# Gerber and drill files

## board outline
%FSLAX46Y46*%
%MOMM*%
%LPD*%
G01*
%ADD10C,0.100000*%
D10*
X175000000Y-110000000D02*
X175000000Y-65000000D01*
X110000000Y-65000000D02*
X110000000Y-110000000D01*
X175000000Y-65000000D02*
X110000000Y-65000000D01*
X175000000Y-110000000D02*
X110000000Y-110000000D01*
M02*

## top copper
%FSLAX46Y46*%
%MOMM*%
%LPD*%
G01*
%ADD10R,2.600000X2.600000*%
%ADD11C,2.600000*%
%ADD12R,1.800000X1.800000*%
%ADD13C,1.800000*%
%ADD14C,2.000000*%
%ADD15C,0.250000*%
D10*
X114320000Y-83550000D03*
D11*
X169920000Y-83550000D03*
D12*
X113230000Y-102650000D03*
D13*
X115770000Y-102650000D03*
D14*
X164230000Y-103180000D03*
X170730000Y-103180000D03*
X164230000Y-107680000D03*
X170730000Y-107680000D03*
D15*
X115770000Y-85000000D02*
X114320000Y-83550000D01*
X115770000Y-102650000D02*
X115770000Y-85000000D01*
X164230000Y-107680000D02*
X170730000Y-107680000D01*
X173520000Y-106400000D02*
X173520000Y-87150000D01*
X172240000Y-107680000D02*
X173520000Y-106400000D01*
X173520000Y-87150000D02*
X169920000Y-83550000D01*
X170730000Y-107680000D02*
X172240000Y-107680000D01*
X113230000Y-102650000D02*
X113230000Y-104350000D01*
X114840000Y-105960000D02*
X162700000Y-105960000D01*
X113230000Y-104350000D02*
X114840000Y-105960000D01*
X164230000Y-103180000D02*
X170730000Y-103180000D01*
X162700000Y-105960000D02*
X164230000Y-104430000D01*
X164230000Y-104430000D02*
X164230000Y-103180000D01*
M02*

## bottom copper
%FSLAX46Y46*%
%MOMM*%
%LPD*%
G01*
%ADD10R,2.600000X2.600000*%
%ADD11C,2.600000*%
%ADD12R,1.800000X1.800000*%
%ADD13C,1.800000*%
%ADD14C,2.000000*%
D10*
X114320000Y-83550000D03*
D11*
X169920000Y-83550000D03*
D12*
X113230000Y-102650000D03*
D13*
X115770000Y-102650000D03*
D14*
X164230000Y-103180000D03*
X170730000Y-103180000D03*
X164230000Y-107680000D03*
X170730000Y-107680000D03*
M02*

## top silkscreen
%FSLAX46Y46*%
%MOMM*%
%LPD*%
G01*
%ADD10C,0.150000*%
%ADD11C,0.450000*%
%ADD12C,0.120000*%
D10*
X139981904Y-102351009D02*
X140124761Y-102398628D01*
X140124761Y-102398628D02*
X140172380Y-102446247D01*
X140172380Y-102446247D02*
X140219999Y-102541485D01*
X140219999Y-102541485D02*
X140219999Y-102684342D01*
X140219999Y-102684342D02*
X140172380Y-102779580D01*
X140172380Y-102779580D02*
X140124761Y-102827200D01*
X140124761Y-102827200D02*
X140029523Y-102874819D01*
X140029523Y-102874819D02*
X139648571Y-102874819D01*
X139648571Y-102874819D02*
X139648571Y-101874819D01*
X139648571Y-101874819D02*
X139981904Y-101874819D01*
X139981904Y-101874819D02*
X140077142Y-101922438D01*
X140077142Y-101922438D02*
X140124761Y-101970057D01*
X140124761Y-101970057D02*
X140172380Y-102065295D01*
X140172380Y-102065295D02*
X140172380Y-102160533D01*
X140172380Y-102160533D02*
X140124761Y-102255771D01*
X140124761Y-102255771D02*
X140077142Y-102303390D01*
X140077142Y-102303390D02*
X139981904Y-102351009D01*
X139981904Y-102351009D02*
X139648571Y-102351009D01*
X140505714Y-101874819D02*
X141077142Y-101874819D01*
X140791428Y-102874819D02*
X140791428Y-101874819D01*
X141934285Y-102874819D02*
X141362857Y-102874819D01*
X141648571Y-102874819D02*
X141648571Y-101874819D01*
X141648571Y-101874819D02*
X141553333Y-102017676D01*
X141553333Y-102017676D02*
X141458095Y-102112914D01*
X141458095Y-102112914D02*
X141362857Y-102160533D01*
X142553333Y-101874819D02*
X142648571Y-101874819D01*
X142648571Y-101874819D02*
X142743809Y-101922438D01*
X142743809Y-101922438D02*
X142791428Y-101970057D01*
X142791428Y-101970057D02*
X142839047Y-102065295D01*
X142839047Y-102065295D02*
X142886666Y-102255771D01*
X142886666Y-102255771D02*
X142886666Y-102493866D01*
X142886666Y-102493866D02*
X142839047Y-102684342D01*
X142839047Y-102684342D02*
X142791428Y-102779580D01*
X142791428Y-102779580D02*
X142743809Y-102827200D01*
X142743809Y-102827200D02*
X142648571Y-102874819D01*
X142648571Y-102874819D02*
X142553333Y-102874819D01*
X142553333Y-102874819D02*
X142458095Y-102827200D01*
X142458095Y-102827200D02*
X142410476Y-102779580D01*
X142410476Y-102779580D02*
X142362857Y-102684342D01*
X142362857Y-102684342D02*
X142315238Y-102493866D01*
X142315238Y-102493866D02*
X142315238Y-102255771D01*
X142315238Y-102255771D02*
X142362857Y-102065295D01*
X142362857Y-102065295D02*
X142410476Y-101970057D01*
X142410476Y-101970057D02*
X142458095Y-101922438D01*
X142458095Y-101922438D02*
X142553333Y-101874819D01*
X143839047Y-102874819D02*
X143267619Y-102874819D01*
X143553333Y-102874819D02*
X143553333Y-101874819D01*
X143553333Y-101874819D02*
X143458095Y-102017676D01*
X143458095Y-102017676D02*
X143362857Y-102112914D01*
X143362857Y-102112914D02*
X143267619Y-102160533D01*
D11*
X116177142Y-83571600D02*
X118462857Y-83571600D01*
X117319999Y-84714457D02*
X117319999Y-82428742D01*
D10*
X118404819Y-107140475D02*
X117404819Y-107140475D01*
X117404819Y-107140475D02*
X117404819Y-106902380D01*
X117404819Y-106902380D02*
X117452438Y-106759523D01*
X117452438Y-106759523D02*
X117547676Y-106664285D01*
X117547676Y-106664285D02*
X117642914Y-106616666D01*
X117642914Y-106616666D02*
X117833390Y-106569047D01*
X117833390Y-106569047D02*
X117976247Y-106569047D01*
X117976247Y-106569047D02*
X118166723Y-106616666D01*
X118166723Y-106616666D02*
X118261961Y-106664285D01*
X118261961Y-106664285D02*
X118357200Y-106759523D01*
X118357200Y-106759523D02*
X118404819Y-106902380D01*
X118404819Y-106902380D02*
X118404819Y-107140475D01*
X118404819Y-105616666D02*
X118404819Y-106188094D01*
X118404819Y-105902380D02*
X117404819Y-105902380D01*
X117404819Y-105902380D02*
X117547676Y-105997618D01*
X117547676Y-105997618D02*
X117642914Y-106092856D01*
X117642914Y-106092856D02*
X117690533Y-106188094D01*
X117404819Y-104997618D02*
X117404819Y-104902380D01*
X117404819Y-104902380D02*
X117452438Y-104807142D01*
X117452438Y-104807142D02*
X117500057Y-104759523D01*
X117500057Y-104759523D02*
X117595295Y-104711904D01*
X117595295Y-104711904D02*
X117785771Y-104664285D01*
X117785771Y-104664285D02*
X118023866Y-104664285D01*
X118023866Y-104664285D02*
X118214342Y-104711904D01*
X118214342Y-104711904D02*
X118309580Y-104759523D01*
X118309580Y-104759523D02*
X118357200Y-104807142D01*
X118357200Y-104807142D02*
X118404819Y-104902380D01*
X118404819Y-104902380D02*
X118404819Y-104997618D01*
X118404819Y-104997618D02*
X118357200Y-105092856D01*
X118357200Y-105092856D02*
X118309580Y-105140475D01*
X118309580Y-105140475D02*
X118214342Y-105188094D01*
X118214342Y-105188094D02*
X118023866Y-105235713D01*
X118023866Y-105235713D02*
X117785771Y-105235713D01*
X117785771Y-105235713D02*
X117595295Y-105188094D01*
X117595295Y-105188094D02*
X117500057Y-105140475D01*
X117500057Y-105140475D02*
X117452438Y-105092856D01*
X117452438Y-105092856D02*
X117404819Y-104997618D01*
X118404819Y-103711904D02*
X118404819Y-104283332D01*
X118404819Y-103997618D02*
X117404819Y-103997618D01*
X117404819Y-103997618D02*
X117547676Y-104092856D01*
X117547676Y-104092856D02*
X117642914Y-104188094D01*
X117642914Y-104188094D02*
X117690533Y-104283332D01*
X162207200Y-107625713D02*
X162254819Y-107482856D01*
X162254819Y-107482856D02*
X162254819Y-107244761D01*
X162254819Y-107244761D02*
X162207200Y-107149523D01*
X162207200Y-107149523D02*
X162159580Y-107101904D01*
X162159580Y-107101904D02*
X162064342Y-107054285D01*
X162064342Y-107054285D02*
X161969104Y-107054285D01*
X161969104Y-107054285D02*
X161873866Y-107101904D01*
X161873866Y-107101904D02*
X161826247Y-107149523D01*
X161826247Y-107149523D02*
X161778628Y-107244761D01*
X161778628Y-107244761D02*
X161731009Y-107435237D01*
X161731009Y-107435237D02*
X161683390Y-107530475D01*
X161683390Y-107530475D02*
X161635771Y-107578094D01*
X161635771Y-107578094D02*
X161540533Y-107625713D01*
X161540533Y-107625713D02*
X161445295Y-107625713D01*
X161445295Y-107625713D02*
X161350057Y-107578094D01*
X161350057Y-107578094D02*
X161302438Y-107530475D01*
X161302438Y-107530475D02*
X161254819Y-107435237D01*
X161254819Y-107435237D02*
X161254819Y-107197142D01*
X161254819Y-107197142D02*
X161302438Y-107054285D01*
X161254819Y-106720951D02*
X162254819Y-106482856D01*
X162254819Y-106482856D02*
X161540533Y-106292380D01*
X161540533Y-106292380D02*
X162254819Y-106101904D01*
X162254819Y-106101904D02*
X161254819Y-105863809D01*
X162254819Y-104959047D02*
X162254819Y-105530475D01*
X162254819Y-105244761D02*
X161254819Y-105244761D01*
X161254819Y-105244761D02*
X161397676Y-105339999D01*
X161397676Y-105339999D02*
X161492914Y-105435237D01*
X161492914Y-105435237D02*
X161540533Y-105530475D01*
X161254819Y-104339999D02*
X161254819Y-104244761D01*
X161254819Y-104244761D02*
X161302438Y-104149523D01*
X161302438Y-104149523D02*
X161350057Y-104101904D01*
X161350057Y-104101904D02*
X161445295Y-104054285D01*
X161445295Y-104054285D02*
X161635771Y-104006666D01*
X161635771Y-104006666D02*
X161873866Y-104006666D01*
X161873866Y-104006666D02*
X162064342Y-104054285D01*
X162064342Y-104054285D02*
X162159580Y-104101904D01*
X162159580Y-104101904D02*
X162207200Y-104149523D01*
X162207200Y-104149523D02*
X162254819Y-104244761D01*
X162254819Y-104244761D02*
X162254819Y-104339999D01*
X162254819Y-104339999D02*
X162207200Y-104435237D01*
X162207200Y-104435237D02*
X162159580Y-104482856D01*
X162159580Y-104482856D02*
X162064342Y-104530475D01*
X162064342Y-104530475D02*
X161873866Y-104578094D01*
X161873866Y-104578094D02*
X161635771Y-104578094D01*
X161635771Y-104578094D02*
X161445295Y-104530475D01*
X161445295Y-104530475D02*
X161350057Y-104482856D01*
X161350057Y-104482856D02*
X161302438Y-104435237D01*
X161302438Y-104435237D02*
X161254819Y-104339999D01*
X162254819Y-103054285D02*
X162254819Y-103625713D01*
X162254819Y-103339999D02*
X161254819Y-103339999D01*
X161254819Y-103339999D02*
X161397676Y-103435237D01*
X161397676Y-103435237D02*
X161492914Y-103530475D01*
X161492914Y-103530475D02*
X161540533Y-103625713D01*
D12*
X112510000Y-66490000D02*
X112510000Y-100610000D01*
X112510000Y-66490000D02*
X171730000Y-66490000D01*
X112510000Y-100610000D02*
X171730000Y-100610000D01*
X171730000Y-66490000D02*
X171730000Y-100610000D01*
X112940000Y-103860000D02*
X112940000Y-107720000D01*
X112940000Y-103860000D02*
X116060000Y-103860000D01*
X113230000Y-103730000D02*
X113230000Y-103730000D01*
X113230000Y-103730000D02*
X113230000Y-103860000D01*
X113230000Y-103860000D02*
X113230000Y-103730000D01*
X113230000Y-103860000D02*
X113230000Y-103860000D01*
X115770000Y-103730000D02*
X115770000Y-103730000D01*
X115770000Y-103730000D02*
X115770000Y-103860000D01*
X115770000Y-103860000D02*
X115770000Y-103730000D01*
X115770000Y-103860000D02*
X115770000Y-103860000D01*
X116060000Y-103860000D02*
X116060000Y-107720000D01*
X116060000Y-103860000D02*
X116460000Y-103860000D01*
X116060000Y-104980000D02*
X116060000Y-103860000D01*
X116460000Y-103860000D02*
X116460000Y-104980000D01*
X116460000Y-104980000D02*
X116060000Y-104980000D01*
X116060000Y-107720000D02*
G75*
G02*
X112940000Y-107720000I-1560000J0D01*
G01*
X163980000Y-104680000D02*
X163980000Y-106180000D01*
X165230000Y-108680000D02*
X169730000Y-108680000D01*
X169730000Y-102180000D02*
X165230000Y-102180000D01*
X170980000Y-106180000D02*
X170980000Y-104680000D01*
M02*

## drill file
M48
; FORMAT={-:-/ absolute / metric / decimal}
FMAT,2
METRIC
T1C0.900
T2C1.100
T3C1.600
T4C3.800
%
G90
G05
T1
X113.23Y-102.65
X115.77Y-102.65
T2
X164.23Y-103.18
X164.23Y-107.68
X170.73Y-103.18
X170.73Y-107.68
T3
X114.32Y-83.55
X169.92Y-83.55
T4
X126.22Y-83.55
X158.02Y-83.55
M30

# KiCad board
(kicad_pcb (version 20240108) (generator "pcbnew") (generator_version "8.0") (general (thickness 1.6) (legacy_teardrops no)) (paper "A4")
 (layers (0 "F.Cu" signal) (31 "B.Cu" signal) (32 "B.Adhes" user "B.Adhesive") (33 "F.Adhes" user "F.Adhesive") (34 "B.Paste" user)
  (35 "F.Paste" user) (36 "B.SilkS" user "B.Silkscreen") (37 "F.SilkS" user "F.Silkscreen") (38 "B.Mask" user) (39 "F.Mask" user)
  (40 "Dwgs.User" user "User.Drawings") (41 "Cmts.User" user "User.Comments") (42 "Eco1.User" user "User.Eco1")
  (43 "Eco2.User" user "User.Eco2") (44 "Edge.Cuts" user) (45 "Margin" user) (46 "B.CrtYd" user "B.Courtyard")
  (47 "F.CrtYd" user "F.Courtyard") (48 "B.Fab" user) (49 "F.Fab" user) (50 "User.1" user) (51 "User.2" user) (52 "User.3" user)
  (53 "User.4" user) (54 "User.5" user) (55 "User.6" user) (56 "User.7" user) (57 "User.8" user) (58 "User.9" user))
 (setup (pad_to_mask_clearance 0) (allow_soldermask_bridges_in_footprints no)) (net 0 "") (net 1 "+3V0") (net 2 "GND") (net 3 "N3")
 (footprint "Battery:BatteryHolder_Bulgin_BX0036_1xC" (layer "F.Cu") (at 114.32 83.55)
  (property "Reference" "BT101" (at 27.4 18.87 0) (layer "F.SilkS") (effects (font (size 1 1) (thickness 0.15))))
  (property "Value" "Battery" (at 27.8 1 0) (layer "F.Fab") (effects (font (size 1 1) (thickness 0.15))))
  (fp_line (start -1.81 -17.06) (end -1.81 17.06) (stroke (width 0.12) (type solid)) (layer "F.SilkS"))
  (fp_line (start -1.81 -17.06) (end 57.41 -17.06) (stroke (width 0.12) (type solid)) (layer "F.SilkS"))
  (fp_line (start -1.81 17.06) (end 57.41 17.06) (stroke (width 0.12) (type solid)) (layer "F.SilkS"))
  (fp_line (start 57.41 -17.06) (end 57.41 17.06) (stroke (width 0.12) (type solid)) (layer "F.SilkS"))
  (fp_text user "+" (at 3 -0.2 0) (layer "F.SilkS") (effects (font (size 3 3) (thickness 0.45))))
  (pad "" np_thru_hole circle (at 11.9 0) (size 3.8 3.8) (drill 3.8) (layers "*.Cu" "*.Mask"))
  (pad "" np_thru_hole circle (at 43.7 0) (size 3.8 3.8) (drill 3.8) (layers "*.Cu" "*.Mask"))
  (pad "1" thru_hole rect (at 0 0) (size 2.6 2.6) (drill 1.6) (layers "*.Cu" "*.Mask") (remove_unused_layers no) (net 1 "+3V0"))
  (pad "2" thru_hole circle (at 55.6 0) (size 2.6 2.6) (drill 1.6) (layers "*.Cu" "*.Mask") (remove_unused_layers no) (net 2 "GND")))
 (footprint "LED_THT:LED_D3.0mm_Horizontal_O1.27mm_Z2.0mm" (layer "F.Cu") (at 113.23 102.65)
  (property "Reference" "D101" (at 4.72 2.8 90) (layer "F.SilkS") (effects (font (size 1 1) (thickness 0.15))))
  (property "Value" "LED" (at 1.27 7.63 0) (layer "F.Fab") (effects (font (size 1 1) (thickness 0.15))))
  (fp_line (start -0.29 1.21) (end -0.29 5.07) (stroke (width 0.12) (type solid)) (layer "F.SilkS"))
  (fp_line (start -0.29 1.21) (end 2.83 1.21) (stroke (width 0.12) (type solid)) (layer "F.SilkS"))
  (fp_line (start 0 1.08) (end 0 1.08) (stroke (width 0.12) (type solid)) (layer "F.SilkS"))
  (fp_line (start 0 1.08) (end 0 1.21) (stroke (width 0.12) (type solid)) (layer "F.SilkS"))
  (fp_line (start 0 1.21) (end 0 1.08) (stroke (width 0.12) (type solid)) (layer "F.SilkS"))
  (fp_line (start 0 1.21) (end 0 1.21) (stroke (width 0.12) (type solid)) (layer "F.SilkS"))
  (fp_line (start 2.54 1.08) (end 2.54 1.08) (stroke (width 0.12) (type solid)) (layer "F.SilkS"))
  (fp_line (start 2.54 1.08) (end 2.54 1.21) (stroke (width 0.12) (type solid)) (layer "F.SilkS"))
  (fp_line (start 2.54 1.21) (end 2.54 1.08) (stroke (width 0.12) (type solid)) (layer "F.SilkS"))
  (fp_line (start 2.54 1.21) (end 2.54 1.21) (stroke (width 0.12) (type solid)) (layer "F.SilkS"))
  (fp_line (start 2.83 1.21) (end 2.83 5.07) (stroke (width 0.12) (type solid)) (layer "F.SilkS"))
  (fp_line (start 2.83 1.21) (end 3.23 1.21) (stroke (width 0.12) (type solid)) (layer "F.SilkS"))
  (fp_line (start 2.83 2.33) (end 2.83 1.21) (stroke (width 0.12) (type solid)) (layer "F.SilkS"))
  (fp_line (start 3.23 1.21) (end 3.23 2.33) (stroke (width 0.12) (type solid)) (layer "F.SilkS"))
  (fp_line (start 3.23 2.33) (end 2.83 2.33) (stroke (width 0.12) (type solid)) (layer "F.SilkS"))
  (fp_arc (start 2.83 5.07) (mid 1.27 6.63) (end -0.29 5.07) (stroke (width 0.12) (type solid)) (layer "F.SilkS"))
  (pad "1" thru_hole rect (at 0 0) (size 1.8 1.8) (drill 0.9) (layers "*.Cu" "*.Mask") (remove_unused_layers no) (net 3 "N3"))
  (pad "2" thru_hole circle (at 2.54 0) (size 1.8 1.8) (drill 0.9) (layers "*.Cu" "*.Mask") (remove_unused_layers no) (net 1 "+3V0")))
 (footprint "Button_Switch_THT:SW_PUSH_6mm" (layer "F.Cu") (at 164.23 103.18)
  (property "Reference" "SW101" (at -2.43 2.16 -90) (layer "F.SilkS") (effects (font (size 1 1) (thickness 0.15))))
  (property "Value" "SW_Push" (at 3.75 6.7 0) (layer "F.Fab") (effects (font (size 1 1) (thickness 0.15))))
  (fp_line (start -0.25 1.5) (end -0.25 3) (stroke (width 0.12) (type solid)) (layer "F.SilkS"))
  (fp_line (start 1 5.5) (end 5.5 5.5) (stroke (width 0.12) (type solid)) (layer "F.SilkS"))
  (fp_line (start 5.5 -1) (end 1 -1) (stroke (width 0.12) (type solid)) (layer "F.SilkS"))
  (fp_line (start 6.75 3) (end 6.75 1.5) (stroke (width 0.12) (type solid)) (layer "F.SilkS"))
  (pad "1" thru_hole circle (at 0 0 90) (size 2 2) (drill 1.1) (layers "*.Cu" "*.Mask") (remove_unused_layers no) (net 3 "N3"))
  (pad "1" thru_hole circle (at 6.5 0 90) (size 2 2) (drill 1.1) (layers "*.Cu" "*.Mask") (remove_unused_layers no) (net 3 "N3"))
  (pad "2" thru_hole circle (at 0 4.5 90) (size 2 2) (drill 1.1) (layers "*.Cu" "*.Mask") (remove_unused_layers no) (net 2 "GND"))
  (pad "2" thru_hole circle (at 6.5 4.5 90) (size 2 2) (drill 1.1) (layers "*.Cu" "*.Mask") (remove_unused_layers no) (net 2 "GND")))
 (gr_line (start 175 110) (end 175 65) (stroke (width 0.1) (type default)) (layer "Edge.Cuts"))
 (gr_line (start 110 65) (end 110 110) (stroke (width 0.1) (type default)) (layer "Edge.Cuts"))
 (gr_line (start 175 65) (end 110 65) (stroke (width 0.1) (type default)) (layer "Edge.Cuts"))
 (gr_line (start 175 110) (end 110 110) (stroke (width 0.1) (type default)) (layer "Edge.Cuts"))
 (segment (start 115.77 85) (end 114.32 83.55) (width 0.25) (layer "F.Cu") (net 1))
 (segment (start 115.77 102.65) (end 115.77 85) (width 0.25) (layer "F.Cu") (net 1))
 (segment (start 164.23 107.68) (end 170.73 107.68) (width 0.25) (layer "F.Cu") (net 2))
 (segment (start 173.52 106.4) (end 173.52 87.15) (width 0.25) (layer "F.Cu") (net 2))
 (segment (start 172.24 107.68) (end 173.52 106.4) (width 0.25) (layer "F.Cu") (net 2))
 (segment (start 173.52 87.15) (end 169.92 83.55) (width 0.25) (layer "F.Cu") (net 2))
 (segment (start 170.73 107.68) (end 172.24 107.68) (width 0.25) (layer "F.Cu") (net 2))
 (segment (start 113.23 102.65) (end 113.23 104.35) (width 0.25) (layer "F.Cu") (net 3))
 (segment (start 114.84 105.96) (end 162.7 105.96) (width 0.25) (layer "F.Cu") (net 3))
 (segment (start 113.23 104.35) (end 114.84 105.96) (width 0.25) (layer "F.Cu") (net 3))
 (segment (start 164.23 103.18) (end 170.73 103.18) (width 0.25) (layer "F.Cu") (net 3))
 (segment (start 162.7 105.96) (end 164.23 104.43) (width 0.25) (layer "F.Cu") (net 3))
 (segment (start 164.23 104.43) (end 164.23 103.18) (width 0.25) (layer "F.Cu") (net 3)))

